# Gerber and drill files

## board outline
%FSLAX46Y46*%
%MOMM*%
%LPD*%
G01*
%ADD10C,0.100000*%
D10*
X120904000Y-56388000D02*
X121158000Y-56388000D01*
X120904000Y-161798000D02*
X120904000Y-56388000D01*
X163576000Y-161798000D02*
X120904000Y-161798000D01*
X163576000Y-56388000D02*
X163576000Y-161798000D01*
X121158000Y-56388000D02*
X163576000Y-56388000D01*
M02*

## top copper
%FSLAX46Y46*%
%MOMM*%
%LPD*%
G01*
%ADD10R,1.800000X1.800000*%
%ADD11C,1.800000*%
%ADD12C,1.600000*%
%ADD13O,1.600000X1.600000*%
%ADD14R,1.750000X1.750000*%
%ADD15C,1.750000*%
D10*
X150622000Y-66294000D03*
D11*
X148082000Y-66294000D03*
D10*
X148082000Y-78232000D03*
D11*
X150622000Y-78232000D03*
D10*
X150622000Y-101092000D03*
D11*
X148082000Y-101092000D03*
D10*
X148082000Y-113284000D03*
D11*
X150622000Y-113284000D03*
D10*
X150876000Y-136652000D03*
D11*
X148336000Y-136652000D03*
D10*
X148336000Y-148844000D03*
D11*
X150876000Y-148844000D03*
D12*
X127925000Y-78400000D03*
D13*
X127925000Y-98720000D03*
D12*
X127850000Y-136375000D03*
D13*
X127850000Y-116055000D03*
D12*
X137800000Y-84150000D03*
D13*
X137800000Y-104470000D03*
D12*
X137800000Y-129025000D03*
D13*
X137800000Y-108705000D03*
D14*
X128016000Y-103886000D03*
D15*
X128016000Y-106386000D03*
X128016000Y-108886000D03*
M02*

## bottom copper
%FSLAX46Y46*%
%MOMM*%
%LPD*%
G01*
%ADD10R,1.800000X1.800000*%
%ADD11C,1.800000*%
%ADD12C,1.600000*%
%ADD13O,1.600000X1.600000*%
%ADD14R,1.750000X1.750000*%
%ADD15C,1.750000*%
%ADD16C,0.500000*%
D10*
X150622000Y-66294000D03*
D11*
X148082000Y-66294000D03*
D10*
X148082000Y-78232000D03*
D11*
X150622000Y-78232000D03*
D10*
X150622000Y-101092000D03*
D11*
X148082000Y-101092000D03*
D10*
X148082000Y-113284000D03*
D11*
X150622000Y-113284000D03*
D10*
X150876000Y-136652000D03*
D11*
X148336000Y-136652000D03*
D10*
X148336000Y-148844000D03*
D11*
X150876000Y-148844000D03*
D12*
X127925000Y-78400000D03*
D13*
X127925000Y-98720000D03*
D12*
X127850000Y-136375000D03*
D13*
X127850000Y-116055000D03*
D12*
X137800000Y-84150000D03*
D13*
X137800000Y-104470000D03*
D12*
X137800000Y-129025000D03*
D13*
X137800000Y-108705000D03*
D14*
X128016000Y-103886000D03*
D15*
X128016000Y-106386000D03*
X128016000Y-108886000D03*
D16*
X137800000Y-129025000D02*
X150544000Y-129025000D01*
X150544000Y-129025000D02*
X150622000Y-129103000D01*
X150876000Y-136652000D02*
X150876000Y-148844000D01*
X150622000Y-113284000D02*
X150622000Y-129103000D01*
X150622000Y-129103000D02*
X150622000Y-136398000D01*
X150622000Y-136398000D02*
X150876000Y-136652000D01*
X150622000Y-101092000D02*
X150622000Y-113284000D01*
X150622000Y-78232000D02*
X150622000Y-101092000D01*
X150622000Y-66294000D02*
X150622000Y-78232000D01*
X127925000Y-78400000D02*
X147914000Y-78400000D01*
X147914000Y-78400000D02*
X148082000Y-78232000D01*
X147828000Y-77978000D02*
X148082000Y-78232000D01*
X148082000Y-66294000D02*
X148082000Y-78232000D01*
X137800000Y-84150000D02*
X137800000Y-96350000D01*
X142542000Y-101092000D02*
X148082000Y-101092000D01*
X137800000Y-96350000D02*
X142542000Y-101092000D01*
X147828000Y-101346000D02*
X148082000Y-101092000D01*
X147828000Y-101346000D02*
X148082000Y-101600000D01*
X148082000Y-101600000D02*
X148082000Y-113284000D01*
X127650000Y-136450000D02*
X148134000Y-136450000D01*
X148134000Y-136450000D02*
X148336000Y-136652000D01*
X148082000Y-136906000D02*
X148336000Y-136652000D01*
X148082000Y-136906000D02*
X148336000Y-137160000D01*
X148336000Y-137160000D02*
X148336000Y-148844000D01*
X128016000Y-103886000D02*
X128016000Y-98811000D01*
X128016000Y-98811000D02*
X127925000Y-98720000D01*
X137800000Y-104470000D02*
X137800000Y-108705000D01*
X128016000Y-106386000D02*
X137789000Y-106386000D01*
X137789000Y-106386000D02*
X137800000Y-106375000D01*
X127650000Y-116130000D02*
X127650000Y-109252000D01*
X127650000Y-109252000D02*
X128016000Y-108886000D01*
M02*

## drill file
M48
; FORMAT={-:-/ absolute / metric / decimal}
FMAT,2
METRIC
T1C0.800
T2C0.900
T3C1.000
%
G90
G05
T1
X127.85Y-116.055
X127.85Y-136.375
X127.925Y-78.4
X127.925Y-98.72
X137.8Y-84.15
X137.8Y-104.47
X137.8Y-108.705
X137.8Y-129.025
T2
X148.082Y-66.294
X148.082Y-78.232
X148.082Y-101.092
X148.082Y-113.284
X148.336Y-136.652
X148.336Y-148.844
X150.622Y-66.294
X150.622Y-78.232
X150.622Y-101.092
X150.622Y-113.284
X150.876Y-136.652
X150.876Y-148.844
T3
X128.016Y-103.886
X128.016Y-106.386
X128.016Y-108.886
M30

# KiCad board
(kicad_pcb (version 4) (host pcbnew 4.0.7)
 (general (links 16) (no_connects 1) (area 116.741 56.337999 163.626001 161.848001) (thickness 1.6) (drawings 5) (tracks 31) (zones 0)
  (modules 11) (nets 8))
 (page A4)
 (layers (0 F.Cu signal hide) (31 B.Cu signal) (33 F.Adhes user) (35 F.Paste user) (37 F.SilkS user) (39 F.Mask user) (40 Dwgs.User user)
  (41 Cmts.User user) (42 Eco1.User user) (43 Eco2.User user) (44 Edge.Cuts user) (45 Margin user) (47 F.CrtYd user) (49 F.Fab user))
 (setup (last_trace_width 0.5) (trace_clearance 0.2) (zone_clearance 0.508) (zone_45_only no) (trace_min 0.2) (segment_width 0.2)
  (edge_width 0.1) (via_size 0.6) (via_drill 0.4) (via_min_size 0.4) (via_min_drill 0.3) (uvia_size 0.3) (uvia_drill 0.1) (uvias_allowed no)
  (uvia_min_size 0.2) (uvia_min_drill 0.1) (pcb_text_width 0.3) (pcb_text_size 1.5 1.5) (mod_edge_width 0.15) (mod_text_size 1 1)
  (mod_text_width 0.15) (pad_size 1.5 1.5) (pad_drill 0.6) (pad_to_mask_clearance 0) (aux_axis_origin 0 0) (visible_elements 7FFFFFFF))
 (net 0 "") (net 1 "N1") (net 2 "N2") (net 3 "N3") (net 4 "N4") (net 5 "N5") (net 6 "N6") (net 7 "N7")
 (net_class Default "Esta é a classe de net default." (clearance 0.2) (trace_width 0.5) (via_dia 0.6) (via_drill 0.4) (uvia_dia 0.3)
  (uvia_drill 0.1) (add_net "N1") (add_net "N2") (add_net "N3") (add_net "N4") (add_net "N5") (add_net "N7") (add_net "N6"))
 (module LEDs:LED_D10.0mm (layer F.Cu) (at 150.622 66.294 180)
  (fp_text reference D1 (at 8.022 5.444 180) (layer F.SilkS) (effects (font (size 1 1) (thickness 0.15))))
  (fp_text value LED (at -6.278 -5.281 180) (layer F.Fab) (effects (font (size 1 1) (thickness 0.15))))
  (pad 1 thru_hole rect (at 0 0 180) (size 1.8 1.8) (drill 0.9) (layers *.Cu *.Mask) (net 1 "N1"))
  (pad 2 thru_hole circle (at 2.54 0 180) (size 1.8 1.8) (drill 0.9) (layers *.Cu *.Mask) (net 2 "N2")))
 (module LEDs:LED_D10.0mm (layer F.Cu) (at 148.082 78.232)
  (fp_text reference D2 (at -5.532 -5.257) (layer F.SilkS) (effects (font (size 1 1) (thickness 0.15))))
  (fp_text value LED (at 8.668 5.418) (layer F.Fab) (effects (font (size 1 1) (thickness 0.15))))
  (pad 1 thru_hole rect (at 0 0) (size 1.8 1.8) (drill 0.9) (layers *.Cu *.Mask) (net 2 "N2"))
  (pad 2 thru_hole circle (at 2.54 0) (size 1.8 1.8) (drill 0.9) (layers *.Cu *.Mask) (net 1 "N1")))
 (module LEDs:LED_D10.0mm (layer F.Cu) (at 150.622 101.092 180)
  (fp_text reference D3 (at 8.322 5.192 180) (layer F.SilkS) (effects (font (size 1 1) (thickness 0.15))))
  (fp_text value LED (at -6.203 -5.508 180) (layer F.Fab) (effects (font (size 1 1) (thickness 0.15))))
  (pad 1 thru_hole rect (at 0 0 180) (size 1.8 1.8) (drill 0.9) (layers *.Cu *.Mask) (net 1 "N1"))
  (pad 2 thru_hole circle (at 2.54 0 180) (size 1.8 1.8) (drill 0.9) (layers *.Cu *.Mask) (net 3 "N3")))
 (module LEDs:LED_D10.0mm (layer F.Cu) (at 148.082 113.284)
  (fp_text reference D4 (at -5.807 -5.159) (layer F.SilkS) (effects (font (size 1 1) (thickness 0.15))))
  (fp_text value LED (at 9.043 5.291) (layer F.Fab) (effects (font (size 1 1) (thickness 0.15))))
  (pad 1 thru_hole rect (at 0 0) (size 1.8 1.8) (drill 0.9) (layers *.Cu *.Mask) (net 3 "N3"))
  (pad 2 thru_hole circle (at 2.54 0) (size 1.8 1.8) (drill 0.9) (layers *.Cu *.Mask) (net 1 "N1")))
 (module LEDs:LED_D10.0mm (layer F.Cu) (at 150.876 136.652 180)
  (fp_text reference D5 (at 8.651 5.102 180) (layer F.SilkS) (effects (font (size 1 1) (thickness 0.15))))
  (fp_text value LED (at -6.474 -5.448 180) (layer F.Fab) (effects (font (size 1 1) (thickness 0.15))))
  (pad 1 thru_hole rect (at 0 0 180) (size 1.8 1.8) (drill 0.9) (layers *.Cu *.Mask) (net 1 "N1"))
  (pad 2 thru_hole circle (at 2.54 0 180) (size 1.8 1.8) (drill 0.9) (layers *.Cu *.Mask) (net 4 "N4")))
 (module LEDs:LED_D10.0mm (layer F.Cu) (at 148.336 148.844)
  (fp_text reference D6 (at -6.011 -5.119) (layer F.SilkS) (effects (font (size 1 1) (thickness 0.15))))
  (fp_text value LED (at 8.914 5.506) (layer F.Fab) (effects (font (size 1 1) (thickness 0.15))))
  (pad 1 thru_hole rect (at 0 0) (size 1.8 1.8) (drill 0.9) (layers *.Cu *.Mask) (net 4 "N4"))
  (pad 2 thru_hole circle (at 2.54 0) (size 1.8 1.8) (drill 0.9) (layers *.Cu *.Mask) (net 1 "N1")))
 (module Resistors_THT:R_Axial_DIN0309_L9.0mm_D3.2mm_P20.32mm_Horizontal (layer F.Cu) (at 127.925 78.4 270)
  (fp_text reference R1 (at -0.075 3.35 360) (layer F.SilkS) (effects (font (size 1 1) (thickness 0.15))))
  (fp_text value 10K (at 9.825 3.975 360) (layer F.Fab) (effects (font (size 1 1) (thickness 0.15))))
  (pad 1 thru_hole circle (at 0 0 270) (size 1.6 1.6) (drill 0.8) (layers *.Cu *.Mask) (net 2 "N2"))
  (pad 2 thru_hole oval (at 20.32 0 270) (size 1.6 1.6) (drill 0.8) (layers *.Cu *.Mask) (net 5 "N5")))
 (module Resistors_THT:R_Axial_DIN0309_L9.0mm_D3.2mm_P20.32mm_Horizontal (layer F.Cu) (at 127.85 136.375 90)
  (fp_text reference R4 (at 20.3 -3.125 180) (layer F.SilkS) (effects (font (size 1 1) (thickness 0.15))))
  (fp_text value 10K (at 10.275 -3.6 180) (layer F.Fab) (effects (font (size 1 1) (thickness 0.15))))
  (pad 1 thru_hole circle (at 0 0 90) (size 1.6 1.6) (drill 0.8) (layers *.Cu *.Mask) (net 4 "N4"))
  (pad 2 thru_hole oval (at 20.32 0 90) (size 1.6 1.6) (drill 0.8) (layers *.Cu *.Mask) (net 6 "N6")))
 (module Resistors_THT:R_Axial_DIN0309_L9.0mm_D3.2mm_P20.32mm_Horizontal (layer F.Cu) (at 137.8 84.15 270)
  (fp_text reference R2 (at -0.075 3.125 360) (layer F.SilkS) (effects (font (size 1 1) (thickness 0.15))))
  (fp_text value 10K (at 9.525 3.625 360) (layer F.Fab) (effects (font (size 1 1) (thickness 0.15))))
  (pad 1 thru_hole circle (at 0 0 270) (size 1.6 1.6) (drill 0.8) (layers *.Cu *.Mask) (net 3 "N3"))
  (pad 2 thru_hole oval (at 20.32 0 270) (size 1.6 1.6) (drill 0.8) (layers *.Cu *.Mask) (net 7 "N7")))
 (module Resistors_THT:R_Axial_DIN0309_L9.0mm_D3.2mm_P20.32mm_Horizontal (layer F.Cu) (at 137.8 129.025 90)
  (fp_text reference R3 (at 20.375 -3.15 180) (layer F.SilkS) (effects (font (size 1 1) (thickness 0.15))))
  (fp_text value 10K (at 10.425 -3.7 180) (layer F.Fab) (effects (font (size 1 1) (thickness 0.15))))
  (pad 1 thru_hole circle (at 0 0 90) (size 1.6 1.6) (drill 0.8) (layers *.Cu *.Mask) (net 1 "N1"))
  (pad 2 thru_hole oval (at 20.32 0 90) (size 1.6 1.6) (drill 0.8) (layers *.Cu *.Mask) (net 7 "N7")))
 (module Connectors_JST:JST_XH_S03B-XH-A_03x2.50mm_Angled (layer F.Cu) (at 128.016 103.886 270)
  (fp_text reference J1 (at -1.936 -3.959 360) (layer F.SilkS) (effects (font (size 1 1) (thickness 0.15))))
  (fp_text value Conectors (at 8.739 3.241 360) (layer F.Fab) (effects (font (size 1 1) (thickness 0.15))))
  (pad 1 thru_hole rect (at 0 0 270) (size 1.75 1.75) (drill 1) (layers *.Cu *.Mask F.SilkS) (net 5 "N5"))
  (pad 2 thru_hole circle (at 2.5 0 270) (size 1.75 1.75) (drill 1) (layers *.Cu *.Mask F.SilkS) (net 7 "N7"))
  (pad 3 thru_hole circle (at 5 0 270) (size 1.75 1.75) (drill 1) (layers *.Cu *.Mask F.SilkS) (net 6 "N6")))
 (gr_line (start 120.904 56.388) (end 121.158 56.388) (angle 90) (layer Edge.Cuts) (width 0.1))
 (gr_line (start 120.904 161.798) (end 120.904 56.388) (angle 90) (layer Edge.Cuts) (width 0.1))
 (gr_line (start 163.576 161.798) (end 120.904 161.798) (angle 90) (layer Edge.Cuts) (width 0.1))
 (gr_line (start 163.576 56.388) (end 163.576 161.798) (angle 90) (layer Edge.Cuts) (width 0.1))
 (gr_line (start 121.158 56.388) (end 163.576 56.388) (angle 90) (layer Edge.Cuts) (width 0.1))
 (segment (start 137.8 129.025) (end 150.544 129.025) (width 0.5) (layer B.Cu) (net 1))
 (segment (start 150.544 129.025) (end 150.622 129.103) (width 0.5) (layer B.Cu) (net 1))
 (segment (start 150.876 136.652) (end 150.876 148.844) (width 0.5) (layer B.Cu) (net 1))
 (segment (start 150.622 113.284) (end 150.622 129.103) (width 0.5) (layer B.Cu) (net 1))
 (segment (start 150.622 129.103) (end 150.622 136.398) (width 0.5) (layer B.Cu) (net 1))
 (segment (start 150.622 136.398) (end 150.876 136.652) (width 0.5) (layer B.Cu) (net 1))
 (segment (start 150.622 101.092) (end 150.622 113.284) (width 0.5) (layer B.Cu) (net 1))
 (segment (start 150.622 78.232) (end 150.622 101.092) (width 0.5) (layer B.Cu) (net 1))
 (segment (start 150.622 66.294) (end 150.622 78.232) (width 0.5) (layer B.Cu) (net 1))
 (segment (start 127.925 78.4) (end 147.914 78.4) (width 0.5) (layer B.Cu) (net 2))
 (segment (start 147.914 78.4) (end 148.082 78.232) (width 0.5) (layer B.Cu) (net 2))
 (segment (start 147.828 77.978) (end 148.082 78.232) (width 0.5) (layer B.Cu) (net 2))
 (segment (start 148.082 66.294) (end 148.082 78.232) (width 0.5) (layer B.Cu) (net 2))
 (segment (start 137.8 84.15) (end 137.8 96.35) (width 0.5) (layer B.Cu) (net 3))
 (segment (start 142.542 101.092) (end 148.082 101.092) (width 0.5) (layer B.Cu) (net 3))
 (segment (start 137.8 96.35) (end 142.542 101.092) (width 0.5) (layer B.Cu) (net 3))
 (segment (start 147.828 101.346) (end 148.082 101.092) (width 0.5) (layer B.Cu) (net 3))
 (segment (start 147.828 101.346) (end 148.082 101.6) (width 0.5) (layer B.Cu) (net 3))
 (segment (start 148.082 101.6) (end 148.082 113.284) (width 0.5) (layer B.Cu) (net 3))
 (segment (start 127.65 136.45) (end 148.134 136.45) (width 0.5) (layer B.Cu) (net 4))
 (segment (start 148.134 136.45) (end 148.336 136.652) (width 0.5) (layer B.Cu) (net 4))
 (segment (start 148.082 136.906) (end 148.336 136.652) (width 0.5) (layer B.Cu) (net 4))
 (segment (start 148.082 136.906) (end 148.336 137.16) (width 0.5) (layer B.Cu) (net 4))
 (segment (start 148.336 137.16) (end 148.336 148.844) (width 0.5) (layer B.Cu) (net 4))
 (segment (start 128.016 103.886) (end 128.016 98.811) (width 0.5) (layer B.Cu) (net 5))
 (segment (start 128.016 98.811) (end 127.925 98.72) (width 0.5) (layer B.Cu) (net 5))
 (segment (start 137.8 104.47) (end 137.8 108.705) (width 0.5) (layer B.Cu) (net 7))
 (segment (start 128.016 106.386) (end 137.789 106.386) (width 0.5) (layer B.Cu) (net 7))
 (segment (start 137.789 106.386) (end 137.8 106.375) (width 0.5) (layer B.Cu) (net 7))
 (segment (start 127.65 116.13) (end 127.65 109.252) (width 0.5) (layer B.Cu) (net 6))
 (segment (start 127.65 109.252) (end 128.016 108.886) (width 0.5) (layer B.Cu) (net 6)))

